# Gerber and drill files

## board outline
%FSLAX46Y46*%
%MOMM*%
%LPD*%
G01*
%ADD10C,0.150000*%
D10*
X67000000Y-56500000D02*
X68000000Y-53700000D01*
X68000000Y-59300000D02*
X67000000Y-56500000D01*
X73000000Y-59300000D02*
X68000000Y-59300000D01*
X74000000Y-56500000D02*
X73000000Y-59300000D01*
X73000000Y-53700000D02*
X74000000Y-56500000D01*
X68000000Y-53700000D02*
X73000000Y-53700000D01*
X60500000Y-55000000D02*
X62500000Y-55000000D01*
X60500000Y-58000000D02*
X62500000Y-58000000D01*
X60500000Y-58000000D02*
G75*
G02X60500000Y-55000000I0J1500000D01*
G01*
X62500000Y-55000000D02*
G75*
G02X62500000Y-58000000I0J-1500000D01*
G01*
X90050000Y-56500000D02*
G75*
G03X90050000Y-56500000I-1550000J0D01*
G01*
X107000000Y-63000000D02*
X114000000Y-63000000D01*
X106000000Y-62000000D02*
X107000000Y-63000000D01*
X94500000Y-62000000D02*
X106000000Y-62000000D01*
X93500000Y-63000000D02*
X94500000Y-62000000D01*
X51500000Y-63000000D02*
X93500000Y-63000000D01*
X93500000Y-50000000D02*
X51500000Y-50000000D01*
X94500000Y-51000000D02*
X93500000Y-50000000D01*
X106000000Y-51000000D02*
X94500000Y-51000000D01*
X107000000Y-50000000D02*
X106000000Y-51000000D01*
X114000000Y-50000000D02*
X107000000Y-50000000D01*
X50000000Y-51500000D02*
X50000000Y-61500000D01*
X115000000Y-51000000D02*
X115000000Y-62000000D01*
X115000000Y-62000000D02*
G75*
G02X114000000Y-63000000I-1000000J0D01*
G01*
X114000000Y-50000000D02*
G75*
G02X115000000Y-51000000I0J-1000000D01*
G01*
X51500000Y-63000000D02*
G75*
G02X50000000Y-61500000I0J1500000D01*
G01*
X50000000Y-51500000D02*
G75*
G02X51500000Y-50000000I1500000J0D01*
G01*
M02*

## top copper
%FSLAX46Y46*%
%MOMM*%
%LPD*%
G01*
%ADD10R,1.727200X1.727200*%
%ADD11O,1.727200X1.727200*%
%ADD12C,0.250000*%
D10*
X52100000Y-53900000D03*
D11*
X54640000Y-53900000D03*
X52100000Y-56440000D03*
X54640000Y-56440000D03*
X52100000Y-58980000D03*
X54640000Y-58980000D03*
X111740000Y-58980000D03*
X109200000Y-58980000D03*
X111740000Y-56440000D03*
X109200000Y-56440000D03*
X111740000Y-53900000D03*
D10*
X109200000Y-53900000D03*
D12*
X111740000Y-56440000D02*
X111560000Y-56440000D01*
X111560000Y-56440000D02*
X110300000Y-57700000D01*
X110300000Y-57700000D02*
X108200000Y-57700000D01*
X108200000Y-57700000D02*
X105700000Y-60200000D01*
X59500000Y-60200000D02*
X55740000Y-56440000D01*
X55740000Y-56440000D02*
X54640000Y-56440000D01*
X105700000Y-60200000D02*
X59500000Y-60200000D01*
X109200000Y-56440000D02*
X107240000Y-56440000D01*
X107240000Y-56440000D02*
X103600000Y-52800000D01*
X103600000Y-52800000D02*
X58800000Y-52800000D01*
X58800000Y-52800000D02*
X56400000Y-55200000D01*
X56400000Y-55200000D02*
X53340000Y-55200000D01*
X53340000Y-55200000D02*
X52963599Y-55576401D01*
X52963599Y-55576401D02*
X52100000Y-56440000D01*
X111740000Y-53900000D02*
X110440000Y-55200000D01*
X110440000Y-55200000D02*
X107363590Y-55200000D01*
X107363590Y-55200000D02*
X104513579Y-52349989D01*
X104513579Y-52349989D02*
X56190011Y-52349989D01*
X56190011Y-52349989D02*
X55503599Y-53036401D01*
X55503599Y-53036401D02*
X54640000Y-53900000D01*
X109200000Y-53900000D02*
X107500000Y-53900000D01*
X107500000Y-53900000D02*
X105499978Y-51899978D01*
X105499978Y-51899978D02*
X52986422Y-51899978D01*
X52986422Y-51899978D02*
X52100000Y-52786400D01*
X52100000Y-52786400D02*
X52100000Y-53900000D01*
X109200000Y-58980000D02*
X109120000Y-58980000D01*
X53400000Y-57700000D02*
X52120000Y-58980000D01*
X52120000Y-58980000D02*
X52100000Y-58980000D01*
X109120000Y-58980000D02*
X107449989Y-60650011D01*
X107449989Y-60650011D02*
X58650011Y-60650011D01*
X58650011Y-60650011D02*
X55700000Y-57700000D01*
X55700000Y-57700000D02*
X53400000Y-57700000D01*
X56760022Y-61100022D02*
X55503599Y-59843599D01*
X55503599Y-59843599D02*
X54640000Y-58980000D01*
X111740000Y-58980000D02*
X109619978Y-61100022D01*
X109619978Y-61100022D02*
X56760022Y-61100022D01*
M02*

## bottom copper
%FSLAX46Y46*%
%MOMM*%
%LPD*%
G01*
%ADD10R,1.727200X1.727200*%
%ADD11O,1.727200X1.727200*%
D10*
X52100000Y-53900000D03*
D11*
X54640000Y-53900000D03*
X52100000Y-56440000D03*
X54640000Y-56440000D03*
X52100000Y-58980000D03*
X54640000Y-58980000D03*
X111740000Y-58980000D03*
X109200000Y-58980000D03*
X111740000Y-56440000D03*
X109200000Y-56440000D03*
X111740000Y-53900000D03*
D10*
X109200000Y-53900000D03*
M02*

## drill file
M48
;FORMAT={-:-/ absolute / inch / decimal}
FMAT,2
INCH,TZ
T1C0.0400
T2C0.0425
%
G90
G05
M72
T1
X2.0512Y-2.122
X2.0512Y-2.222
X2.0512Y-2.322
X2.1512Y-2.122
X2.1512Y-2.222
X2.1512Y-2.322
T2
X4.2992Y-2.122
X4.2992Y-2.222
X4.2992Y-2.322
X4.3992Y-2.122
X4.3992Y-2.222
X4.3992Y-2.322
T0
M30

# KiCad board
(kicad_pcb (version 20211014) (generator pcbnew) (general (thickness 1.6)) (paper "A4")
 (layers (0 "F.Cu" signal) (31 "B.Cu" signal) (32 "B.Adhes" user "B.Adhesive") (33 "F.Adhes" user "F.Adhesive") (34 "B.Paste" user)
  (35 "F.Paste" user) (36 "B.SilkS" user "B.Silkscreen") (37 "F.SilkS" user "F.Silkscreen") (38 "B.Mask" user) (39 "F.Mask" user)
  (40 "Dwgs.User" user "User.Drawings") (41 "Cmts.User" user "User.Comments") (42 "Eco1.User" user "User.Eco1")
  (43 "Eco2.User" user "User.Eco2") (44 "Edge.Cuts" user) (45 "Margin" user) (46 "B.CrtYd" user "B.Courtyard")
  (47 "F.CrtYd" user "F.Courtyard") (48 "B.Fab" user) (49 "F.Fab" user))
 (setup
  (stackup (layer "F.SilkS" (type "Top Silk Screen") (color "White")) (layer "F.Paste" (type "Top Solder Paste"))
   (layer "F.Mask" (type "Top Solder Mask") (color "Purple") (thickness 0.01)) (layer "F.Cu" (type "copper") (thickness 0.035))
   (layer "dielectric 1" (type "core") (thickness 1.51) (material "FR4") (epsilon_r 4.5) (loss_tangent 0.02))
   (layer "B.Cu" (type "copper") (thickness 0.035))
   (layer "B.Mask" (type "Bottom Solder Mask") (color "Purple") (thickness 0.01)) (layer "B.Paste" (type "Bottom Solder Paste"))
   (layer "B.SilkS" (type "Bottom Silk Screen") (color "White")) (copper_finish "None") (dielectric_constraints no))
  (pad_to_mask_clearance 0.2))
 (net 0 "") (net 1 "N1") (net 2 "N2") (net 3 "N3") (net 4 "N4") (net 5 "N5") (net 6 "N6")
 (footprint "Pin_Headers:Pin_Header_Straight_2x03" (layer "F.Cu") (at 52.1 53.9)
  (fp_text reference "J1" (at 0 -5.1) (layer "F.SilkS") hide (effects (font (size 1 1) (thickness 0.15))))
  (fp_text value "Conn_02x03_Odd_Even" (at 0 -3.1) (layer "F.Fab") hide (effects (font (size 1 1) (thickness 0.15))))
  (pad "1" thru_hole rect locked (at 0 0) (size 1.7272 1.7272) (drill 1.016) (layers *.Cu *.Mask) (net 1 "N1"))
  (pad "2" thru_hole oval locked (at 2.54 0) (size 1.7272 1.7272) (drill 1.016) (layers *.Cu *.Mask) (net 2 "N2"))
  (pad "3" thru_hole oval locked (at 0 2.54) (size 1.7272 1.7272) (drill 1.016) (layers *.Cu *.Mask) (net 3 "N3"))
  (pad "4" thru_hole oval locked (at 2.54 2.54) (size 1.7272 1.7272) (drill 1.016) (layers *.Cu *.Mask) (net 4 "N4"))
  (pad "5" thru_hole oval locked (at 0 5.08) (size 1.7272 1.7272) (drill 1.016) (layers *.Cu *.Mask) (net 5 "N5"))
  (pad "6" thru_hole oval locked (at 2.54 5.08) (size 1.7272 1.7272) (drill 1.016) (layers *.Cu *.Mask) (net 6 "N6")))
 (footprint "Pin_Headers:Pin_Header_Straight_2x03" (layer "F.Cu") (at 109.2 53.9)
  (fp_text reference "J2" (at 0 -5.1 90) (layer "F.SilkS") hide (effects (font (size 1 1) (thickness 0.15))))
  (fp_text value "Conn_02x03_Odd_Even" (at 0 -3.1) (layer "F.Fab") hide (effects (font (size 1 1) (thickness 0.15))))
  (pad "1" thru_hole rect locked (at 0 0) (size 1.7272 1.7272) (drill 1.08) (layers *.Cu *.Mask) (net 1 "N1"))
  (pad "2" thru_hole oval locked (at 2.54 0) (size 1.7272 1.7272) (drill 1.08) (layers *.Cu *.Mask) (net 2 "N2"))
  (pad "3" thru_hole oval locked (at 0 2.54) (size 1.7272 1.7272) (drill 1.08) (layers *.Cu *.Mask) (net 3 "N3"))
  (pad "4" thru_hole oval locked (at 2.54 2.54) (size 1.7272 1.7272) (drill 1.08) (layers *.Cu *.Mask) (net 4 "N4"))
  (pad "5" thru_hole oval locked (at 0 5.08) (size 1.7272 1.7272) (drill 1.08) (layers *.Cu *.Mask) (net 5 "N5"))
  (pad "6" thru_hole oval locked (at 2.54 5.08) (size 1.7272 1.7272) (drill 1.08) (layers *.Cu *.Mask) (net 6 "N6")))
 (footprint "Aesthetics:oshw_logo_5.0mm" (layer "F.Cu") (at 100.5 56.5 -90)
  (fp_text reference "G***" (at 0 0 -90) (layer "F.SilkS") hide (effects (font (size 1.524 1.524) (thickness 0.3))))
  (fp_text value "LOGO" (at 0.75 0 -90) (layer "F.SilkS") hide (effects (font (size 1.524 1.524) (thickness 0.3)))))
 (gr_arc (start 60.5 58) (mid 59 56.5) (end 60.5 55) (layer "Edge.Cuts") (width 0.15))
 (gr_line (start 68 59.3) (end 67 56.5) (layer "Edge.Cuts") (width 0.15))
 (gr_line (start 50 51.5) (end 50 61.5) (layer "Edge.Cuts") (width 0.15))
 (gr_line (start 93.5 63) (end 94.5 62) (layer "Edge.Cuts") (width 0.15))
 (gr_circle (center 88.5 56.5) (end 90.05 56.5) (layer "Edge.Cuts") (width 0.15) (fill none))
 (gr_arc (start 115 62) (mid 114.707107 62.707107) (end 114 63) (layer "Edge.Cuts") (width 0.15))
 (gr_line (start 94.5 62) (end 106 62) (layer "Edge.Cuts") (width 0.15))
 (gr_line (start 73 59.3) (end 68 59.3) (layer "Edge.Cuts") (width 0.15))
 (gr_arc (start 50 51.5) (mid 50.43934 50.43934) (end 51.5 50) (layer "Edge.Cuts") (width 0.15))
 (gr_arc (start 62.5 55) (mid 64 56.5) (end 62.5 58) (layer "Edge.Cuts") (width 0.15))
 (gr_line (start 94.5 51) (end 93.5 50) (layer "Edge.Cuts") (width 0.15))
 (gr_line (start 74 56.5) (end 73 59.3) (layer "Edge.Cuts") (width 0.15))
 (gr_line (start 93.5 50) (end 51.5 50) (layer "Edge.Cuts") (width 0.15))
 (gr_line (start 107 50) (end 106 51) (layer "Edge.Cuts") (width 0.15))
 (gr_line (start 114 50) (end 107 50) (layer "Edge.Cuts") (width 0.15))
 (gr_line (start 67 56.5) (end 68 53.7) (layer "Edge.Cuts") (width 0.15))
 (gr_line (start 60.5 58) (end 62.5 58) (layer "Edge.Cuts") (width 0.15))
 (gr_line (start 106 51) (end 94.5 51) (layer "Edge.Cuts") (width 0.15))
 (gr_line (start 68 53.7) (end 73 53.7) (layer "Edge.Cuts") (width 0.15))
 (gr_line (start 60.5 55) (end 62.5 55) (layer "Edge.Cuts") (width 0.15))
 (gr_arc (start 114 50) (mid 114.707107 50.292893) (end 115 51) (layer "Edge.Cuts") (width 0.15))
 (gr_line (start 106 62) (end 107 63) (layer "Edge.Cuts") (width 0.15))
 (gr_arc (start 51.5 63) (mid 50.43934 62.56066) (end 50 61.5) (layer "Edge.Cuts") (width 0.15))
 (gr_line (start 107 63) (end 114 63) (layer "Edge.Cuts") (width 0.15))
 (gr_line (start 73 53.7) (end 74 56.5) (layer "Edge.Cuts") (width 0.15))
 (gr_line (start 51.5 63) (end 93.5 63) (layer "Edge.Cuts") (width 0.15))
 (gr_line (start 115 51) (end 115 62) (layer "Edge.Cuts") (width 0.15))
 (segment (start 55.74 56.44) (end 54.64 56.44) (width 0.25) (layer "F.Cu") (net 4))
 (segment (start 111.56 56.44) (end 110.3 57.7) (width 0.25) (layer "F.Cu") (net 4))
 (segment (start 59.5 60.2) (end 55.74 56.44) (width 0.25) (layer "F.Cu") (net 4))
 (segment (start 108.2 57.7) (end 105.7 60.2) (width 0.25) (layer "F.Cu") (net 4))
 (segment (start 105.7 60.2) (end 59.5 60.2) (width 0.25) (layer "F.Cu") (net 4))
 (segment (start 111.74 56.44) (end 111.56 56.44) (width 0.25) (layer "F.Cu") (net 4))
 (segment (start 110.3 57.7) (end 108.2 57.7) (width 0.25) (layer "F.Cu") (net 4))
 (segment (start 103.6 52.8) (end 58.8 52.8) (width 0.25) (layer "F.Cu") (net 3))
 (segment (start 109.2 56.44) (end 107.24 56.44) (width 0.25) (layer "F.Cu") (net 3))
 (segment (start 53.34 55.2) (end 52.963599 55.576401) (width 0.25) (layer "F.Cu") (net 3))
 (segment (start 56.4 55.2) (end 53.34 55.2) (width 0.25) (layer "F.Cu") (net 3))
 (segment (start 107.24 56.44) (end 103.6 52.8) (width 0.25) (layer "F.Cu") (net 3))
 (segment (start 52.963599 55.576401) (end 52.1 56.44) (width 0.25) (layer "F.Cu") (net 3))
 (segment (start 58.8 52.8) (end 56.4 55.2) (width 0.25) (layer "F.Cu") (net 3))
 (segment (start 111.74 53.9) (end 110.44 55.2) (width 0.25) (layer "F.Cu") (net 2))
 (segment (start 56.190011 52.349989) (end 55.503599 53.036401) (width 0.25) (layer "F.Cu") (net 2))
 (segment (start 104.513579 52.349989) (end 56.190011 52.349989) (width 0.25) (layer "F.Cu") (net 2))
 (segment (start 107.36359 55.2) (end 104.513579 52.349989) (width 0.25) (layer "F.Cu") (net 2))
 (segment (start 55.503599 53.036401) (end 54.64 53.9) (width 0.25) (layer "F.Cu") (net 2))
 (segment (start 110.44 55.2) (end 107.36359 55.2) (width 0.25) (layer "F.Cu") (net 2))
 (segment (start 105.499978 51.899978) (end 52.986422 51.899978) (width 0.25) (layer "F.Cu") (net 1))
 (segment (start 52.986422 51.899978) (end 52.1 52.7864) (width 0.25) (layer "F.Cu") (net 1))
 (segment (start 52.1 52.7864) (end 52.1 53.9) (width 0.25) (layer "F.Cu") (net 1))
 (segment (start 107.5 53.9) (end 105.499978 51.899978) (width 0.25) (layer "F.Cu") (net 1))
 (segment (start 109.2 53.9) (end 107.5 53.9) (width 0.25) (layer "F.Cu") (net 1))
 (segment (start 107.449989 60.650011) (end 58.650011 60.650011) (width 0.25) (layer "F.Cu") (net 5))
 (segment (start 109.2 58.98) (end 109.12 58.98) (width 0.25) (layer "F.Cu") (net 5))
 (segment (start 58.650011 60.650011) (end 55.7 57.7) (width 0.25) (layer "F.Cu") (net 5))
 (segment (start 109.12 58.98) (end 107.449989 60.650011) (width 0.25) (layer "F.Cu") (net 5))
 (segment (start 55.7 57.7) (end 53.4 57.7) (width 0.25) (layer "F.Cu") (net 5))
 (segment (start 53.4 57.7) (end 52.12 58.98) (width 0.25) (layer "F.Cu") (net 5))
 (segment (start 52.12 58.98) (end 52.1 58.98) (width 0.25) (layer "F.Cu") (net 5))
 (segment (start 109.619978 61.100022) (end 56.760022 61.100022) (width 0.25) (layer "F.Cu") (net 6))
 (segment (start 111.74 58.98) (end 109.619978 61.100022) (width 0.25) (layer "F.Cu") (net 6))
 (segment (start 56.760022 61.100022) (end 55.503599 59.843599) (width 0.25) (layer "F.Cu") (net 6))
 (segment (start 55.503599 59.843599) (end 54.64 58.98) (width 0.25) (layer "F.Cu") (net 6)))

